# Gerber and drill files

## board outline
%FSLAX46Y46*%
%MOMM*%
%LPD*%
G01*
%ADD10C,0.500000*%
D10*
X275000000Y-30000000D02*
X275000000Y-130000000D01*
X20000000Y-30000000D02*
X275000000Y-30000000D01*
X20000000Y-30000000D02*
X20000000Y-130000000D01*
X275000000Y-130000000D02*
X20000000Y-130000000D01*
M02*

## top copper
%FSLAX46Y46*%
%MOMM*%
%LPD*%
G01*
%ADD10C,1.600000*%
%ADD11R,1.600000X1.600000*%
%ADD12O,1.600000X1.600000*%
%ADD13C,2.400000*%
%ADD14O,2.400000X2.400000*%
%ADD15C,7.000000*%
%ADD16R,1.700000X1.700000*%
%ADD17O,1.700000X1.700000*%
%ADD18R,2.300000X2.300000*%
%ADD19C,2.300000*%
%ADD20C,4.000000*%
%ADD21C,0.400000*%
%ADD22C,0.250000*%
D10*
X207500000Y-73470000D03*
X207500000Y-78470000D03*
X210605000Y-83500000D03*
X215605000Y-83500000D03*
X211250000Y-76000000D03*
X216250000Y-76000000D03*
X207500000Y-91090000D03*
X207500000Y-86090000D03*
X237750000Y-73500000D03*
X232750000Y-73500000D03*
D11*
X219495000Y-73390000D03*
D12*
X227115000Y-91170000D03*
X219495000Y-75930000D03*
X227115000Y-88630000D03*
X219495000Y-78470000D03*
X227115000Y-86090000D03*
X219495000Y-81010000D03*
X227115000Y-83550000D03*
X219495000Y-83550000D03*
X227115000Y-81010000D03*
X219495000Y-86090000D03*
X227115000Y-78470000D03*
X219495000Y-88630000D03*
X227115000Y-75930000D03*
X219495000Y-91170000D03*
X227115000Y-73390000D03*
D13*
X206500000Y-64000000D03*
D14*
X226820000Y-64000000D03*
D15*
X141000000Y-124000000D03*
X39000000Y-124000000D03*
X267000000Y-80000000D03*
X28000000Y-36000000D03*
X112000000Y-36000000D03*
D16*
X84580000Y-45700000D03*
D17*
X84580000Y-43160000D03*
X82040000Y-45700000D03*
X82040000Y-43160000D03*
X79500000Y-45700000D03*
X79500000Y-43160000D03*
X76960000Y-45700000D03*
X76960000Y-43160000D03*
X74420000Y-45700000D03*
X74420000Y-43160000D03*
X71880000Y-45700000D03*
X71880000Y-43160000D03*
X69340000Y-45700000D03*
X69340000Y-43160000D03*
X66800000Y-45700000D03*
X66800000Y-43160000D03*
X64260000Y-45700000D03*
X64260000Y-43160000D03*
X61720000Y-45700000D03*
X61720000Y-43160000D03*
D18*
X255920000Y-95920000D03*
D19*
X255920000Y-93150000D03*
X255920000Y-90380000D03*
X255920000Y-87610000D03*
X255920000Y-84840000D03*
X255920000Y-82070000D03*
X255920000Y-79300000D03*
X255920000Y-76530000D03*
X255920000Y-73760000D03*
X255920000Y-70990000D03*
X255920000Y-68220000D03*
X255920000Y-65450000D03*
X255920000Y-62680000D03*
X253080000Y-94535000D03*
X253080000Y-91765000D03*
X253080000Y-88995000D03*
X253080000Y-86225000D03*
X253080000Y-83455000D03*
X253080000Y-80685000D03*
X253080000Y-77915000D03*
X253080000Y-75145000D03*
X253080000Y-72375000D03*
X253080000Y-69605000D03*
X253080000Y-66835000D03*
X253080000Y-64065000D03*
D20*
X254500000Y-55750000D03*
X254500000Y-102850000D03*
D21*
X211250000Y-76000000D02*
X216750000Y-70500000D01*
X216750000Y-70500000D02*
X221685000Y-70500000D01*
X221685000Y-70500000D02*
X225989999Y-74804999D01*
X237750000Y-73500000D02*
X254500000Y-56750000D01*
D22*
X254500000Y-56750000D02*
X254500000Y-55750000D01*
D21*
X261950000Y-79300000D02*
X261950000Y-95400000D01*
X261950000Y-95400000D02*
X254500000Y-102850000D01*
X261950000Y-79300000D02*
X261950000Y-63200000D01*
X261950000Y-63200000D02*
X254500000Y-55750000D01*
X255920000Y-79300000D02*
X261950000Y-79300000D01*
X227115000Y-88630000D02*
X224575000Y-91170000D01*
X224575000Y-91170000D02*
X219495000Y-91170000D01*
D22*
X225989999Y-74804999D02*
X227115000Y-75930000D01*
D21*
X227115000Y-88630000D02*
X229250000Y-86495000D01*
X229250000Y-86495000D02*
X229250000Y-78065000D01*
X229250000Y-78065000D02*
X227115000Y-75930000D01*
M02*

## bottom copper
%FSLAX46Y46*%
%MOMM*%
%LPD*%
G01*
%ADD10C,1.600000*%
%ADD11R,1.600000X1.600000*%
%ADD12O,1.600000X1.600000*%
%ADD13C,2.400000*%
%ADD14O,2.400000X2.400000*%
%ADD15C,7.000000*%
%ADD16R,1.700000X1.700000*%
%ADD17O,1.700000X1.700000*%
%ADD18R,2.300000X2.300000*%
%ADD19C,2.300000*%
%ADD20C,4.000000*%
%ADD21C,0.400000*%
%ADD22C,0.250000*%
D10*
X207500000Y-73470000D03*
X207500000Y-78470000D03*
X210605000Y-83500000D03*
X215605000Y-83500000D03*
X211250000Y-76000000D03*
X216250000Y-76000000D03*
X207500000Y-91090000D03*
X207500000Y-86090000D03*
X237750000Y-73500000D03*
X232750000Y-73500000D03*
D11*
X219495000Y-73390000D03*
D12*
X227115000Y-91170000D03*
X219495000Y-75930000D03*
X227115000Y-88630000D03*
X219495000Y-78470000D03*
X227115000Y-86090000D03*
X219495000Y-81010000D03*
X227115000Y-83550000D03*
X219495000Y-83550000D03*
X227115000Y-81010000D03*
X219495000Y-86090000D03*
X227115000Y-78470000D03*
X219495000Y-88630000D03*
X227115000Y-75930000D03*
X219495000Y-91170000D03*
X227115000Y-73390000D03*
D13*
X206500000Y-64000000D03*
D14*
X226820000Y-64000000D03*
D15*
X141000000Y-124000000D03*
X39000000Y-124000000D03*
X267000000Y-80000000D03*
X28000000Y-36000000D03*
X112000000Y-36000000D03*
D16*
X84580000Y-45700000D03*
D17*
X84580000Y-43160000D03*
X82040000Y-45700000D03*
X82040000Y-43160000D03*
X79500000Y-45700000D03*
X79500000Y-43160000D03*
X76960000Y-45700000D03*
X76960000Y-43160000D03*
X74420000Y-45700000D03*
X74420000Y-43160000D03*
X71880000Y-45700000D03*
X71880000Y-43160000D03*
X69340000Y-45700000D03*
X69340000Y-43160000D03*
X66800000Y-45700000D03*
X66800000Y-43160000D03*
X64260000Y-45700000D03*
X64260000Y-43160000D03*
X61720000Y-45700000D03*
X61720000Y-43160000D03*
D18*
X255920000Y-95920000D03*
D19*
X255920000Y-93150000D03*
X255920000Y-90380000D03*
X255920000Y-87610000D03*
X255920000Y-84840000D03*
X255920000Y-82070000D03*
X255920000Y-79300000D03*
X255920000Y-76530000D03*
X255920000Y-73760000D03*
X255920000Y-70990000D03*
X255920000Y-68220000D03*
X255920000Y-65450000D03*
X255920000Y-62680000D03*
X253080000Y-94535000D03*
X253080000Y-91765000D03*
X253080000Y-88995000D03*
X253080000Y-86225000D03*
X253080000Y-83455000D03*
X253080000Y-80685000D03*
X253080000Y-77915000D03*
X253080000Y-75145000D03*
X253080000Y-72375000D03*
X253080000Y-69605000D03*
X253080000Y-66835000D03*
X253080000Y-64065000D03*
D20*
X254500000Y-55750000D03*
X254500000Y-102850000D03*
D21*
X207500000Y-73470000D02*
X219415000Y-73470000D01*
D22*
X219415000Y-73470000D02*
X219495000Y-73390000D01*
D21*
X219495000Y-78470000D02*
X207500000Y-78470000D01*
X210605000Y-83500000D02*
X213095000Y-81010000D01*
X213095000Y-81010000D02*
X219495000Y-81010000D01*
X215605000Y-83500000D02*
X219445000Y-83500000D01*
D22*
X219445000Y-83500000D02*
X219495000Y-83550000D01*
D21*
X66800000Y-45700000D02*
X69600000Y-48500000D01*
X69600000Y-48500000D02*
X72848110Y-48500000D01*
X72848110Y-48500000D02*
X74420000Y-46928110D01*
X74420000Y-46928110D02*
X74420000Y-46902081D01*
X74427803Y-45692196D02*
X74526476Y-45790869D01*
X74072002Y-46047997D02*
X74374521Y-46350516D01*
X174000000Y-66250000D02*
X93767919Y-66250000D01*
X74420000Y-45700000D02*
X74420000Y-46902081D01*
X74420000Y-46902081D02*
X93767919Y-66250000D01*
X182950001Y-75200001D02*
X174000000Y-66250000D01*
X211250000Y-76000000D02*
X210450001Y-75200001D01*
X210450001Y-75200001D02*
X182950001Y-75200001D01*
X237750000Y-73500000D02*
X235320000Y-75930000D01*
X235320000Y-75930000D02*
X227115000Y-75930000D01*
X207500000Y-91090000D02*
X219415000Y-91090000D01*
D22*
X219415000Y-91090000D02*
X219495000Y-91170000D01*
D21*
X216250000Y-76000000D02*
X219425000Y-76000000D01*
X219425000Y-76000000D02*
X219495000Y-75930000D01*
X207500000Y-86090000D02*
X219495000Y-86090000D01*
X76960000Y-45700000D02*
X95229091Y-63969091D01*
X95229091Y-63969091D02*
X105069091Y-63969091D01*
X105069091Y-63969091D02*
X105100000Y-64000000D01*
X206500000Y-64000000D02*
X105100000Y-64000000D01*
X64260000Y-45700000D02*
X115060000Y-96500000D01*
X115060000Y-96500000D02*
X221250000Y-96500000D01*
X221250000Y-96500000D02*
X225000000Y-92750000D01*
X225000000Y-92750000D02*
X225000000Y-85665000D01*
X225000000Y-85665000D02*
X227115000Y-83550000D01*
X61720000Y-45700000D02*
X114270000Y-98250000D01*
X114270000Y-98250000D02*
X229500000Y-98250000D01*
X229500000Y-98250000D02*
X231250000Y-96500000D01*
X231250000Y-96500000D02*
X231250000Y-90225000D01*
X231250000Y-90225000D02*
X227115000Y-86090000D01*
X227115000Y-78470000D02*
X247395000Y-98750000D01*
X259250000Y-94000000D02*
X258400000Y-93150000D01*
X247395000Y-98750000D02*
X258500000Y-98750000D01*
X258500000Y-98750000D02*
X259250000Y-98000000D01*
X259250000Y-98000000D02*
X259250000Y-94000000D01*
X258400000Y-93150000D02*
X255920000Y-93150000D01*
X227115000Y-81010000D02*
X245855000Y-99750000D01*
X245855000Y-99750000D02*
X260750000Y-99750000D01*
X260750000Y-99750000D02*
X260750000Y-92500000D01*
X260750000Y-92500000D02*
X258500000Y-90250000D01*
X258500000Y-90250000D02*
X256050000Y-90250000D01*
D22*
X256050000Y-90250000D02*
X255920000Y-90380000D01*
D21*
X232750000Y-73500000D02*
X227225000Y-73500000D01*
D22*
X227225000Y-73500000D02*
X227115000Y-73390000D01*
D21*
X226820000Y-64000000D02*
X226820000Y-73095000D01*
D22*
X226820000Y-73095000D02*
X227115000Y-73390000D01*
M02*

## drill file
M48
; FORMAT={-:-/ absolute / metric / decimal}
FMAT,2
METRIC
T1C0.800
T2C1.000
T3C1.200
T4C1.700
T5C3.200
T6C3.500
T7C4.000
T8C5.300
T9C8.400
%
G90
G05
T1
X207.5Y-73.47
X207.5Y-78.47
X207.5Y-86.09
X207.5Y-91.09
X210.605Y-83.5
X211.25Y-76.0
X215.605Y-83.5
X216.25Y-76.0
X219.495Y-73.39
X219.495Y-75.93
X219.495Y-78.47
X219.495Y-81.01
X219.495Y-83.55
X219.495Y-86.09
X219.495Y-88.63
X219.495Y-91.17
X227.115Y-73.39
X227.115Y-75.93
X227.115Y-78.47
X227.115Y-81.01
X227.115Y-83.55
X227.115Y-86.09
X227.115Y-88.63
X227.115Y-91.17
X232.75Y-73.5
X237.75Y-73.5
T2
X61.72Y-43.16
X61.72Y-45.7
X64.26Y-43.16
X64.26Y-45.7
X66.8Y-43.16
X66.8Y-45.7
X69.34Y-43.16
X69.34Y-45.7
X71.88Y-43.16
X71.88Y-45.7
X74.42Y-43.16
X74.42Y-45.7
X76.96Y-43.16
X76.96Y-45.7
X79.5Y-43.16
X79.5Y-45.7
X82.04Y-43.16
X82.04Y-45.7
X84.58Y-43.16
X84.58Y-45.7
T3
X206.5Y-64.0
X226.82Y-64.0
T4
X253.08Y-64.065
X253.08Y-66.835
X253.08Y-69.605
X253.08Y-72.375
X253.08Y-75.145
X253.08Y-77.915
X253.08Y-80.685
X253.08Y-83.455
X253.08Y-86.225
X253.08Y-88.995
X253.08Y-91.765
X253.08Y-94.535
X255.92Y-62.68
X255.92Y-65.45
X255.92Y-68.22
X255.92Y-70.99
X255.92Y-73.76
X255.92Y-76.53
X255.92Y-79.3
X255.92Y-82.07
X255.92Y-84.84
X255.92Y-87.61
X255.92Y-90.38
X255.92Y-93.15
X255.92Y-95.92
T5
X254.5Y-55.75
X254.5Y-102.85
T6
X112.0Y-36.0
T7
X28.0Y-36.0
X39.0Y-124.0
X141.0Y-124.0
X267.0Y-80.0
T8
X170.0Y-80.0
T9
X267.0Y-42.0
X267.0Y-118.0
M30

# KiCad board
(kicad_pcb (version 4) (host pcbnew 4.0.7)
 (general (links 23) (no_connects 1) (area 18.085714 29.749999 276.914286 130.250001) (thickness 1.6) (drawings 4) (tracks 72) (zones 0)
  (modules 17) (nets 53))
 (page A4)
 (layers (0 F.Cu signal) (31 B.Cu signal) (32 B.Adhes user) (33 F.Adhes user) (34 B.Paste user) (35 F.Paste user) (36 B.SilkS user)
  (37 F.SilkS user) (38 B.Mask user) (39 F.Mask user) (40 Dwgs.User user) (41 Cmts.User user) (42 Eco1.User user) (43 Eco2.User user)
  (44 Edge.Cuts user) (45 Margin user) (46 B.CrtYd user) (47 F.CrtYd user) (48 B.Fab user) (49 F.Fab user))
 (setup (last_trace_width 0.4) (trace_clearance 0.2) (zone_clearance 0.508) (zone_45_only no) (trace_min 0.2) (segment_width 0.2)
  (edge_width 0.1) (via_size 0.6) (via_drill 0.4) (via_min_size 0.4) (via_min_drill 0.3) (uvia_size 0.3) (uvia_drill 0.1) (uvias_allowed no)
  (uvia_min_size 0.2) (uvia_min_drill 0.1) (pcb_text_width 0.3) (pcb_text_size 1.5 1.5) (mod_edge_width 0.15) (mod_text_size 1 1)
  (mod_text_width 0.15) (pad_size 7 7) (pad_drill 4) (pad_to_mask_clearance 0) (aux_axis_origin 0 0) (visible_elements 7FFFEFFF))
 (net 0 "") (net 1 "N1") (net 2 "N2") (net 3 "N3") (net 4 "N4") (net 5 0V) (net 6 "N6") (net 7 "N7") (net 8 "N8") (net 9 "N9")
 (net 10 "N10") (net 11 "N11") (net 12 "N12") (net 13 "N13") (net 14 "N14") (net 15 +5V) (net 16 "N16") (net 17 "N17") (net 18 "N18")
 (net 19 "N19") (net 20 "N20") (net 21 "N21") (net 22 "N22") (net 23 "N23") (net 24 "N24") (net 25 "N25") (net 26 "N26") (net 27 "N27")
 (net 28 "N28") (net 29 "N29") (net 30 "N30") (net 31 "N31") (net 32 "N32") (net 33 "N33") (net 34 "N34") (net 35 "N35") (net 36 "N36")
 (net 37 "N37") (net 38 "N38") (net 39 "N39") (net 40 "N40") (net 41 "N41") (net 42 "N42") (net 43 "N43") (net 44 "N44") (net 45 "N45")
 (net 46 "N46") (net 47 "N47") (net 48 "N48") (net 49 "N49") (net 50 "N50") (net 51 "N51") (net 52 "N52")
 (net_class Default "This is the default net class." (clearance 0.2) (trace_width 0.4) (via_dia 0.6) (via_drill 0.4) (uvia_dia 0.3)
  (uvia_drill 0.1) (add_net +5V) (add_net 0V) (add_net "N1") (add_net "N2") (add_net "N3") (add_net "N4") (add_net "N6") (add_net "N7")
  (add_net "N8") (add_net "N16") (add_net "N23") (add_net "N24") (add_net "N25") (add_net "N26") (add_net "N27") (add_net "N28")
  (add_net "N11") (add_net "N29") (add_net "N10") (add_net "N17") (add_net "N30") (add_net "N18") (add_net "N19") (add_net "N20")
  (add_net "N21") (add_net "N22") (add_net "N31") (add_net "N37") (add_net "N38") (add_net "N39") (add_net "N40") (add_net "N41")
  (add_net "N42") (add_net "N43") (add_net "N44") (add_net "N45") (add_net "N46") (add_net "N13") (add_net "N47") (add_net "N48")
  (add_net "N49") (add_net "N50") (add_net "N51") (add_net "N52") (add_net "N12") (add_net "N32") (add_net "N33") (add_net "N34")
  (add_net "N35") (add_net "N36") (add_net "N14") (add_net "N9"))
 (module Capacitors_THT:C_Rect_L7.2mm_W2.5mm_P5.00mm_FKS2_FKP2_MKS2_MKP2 (layer F.Cu) (at 207.5 73.47 270)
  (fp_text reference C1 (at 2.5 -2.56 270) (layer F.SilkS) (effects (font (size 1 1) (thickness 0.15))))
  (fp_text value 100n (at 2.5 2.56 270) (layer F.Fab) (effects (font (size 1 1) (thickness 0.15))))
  (pad 1 thru_hole circle (at 0 0 270) (size 1.6 1.6) (drill 0.8) (layers *.Cu *.Mask) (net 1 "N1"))
  (pad 2 thru_hole circle (at 5 0 270) (size 1.6 1.6) (drill 0.8) (layers *.Cu *.Mask) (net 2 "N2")))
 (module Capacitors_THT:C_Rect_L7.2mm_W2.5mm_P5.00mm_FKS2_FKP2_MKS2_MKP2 (layer F.Cu) (at 210.605 83.5)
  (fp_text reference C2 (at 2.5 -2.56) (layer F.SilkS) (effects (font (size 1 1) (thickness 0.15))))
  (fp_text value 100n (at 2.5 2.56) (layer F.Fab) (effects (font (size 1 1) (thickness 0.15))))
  (pad 1 thru_hole circle (at 0 0) (size 1.6 1.6) (drill 0.8) (layers *.Cu *.Mask) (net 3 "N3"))
  (pad 2 thru_hole circle (at 5 0) (size 1.6 1.6) (drill 0.8) (layers *.Cu *.Mask) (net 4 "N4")))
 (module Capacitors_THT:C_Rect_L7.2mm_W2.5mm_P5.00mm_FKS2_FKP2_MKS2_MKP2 (layer F.Cu) (at 211.25 76)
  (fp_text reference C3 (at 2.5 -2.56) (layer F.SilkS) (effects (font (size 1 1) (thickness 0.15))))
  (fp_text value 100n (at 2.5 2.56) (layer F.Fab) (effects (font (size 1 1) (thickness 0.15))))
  (pad 1 thru_hole circle (at 0 0) (size 1.6 1.6) (drill 0.8) (layers *.Cu *.Mask) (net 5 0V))
  (pad 2 thru_hole circle (at 5 0) (size 1.6 1.6) (drill 0.8) (layers *.Cu *.Mask) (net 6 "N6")))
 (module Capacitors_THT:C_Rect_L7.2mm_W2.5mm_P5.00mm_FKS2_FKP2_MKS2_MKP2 (layer F.Cu) (at 207.5 91.09 90)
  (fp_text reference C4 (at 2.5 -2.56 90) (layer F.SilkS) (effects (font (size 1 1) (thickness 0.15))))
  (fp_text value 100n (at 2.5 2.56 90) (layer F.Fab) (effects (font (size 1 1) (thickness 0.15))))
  (pad 1 thru_hole circle (at 0 0 90) (size 1.6 1.6) (drill 0.8) (layers *.Cu *.Mask) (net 5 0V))
  (pad 2 thru_hole circle (at 5 0 90) (size 1.6 1.6) (drill 0.8) (layers *.Cu *.Mask) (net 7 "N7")))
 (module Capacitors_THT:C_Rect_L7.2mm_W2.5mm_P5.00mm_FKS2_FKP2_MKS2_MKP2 (layer F.Cu) (at 237.75 73.5 180)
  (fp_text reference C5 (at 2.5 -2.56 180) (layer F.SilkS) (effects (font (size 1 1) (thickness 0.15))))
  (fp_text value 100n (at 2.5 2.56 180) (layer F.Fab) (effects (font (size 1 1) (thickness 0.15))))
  (pad 1 thru_hole circle (at 0 0 180) (size 1.6 1.6) (drill 0.8) (layers *.Cu *.Mask) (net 5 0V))
  (pad 2 thru_hole circle (at 5 0 180) (size 1.6 1.6) (drill 0.8) (layers *.Cu *.Mask) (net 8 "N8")))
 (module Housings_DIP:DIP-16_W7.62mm (layer F.Cu) (at 219.495 73.39)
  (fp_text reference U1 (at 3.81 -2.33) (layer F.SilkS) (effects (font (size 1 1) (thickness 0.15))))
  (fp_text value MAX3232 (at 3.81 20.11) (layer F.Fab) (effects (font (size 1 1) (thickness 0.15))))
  (pad 1 thru_hole rect (at 0 0) (size 1.6 1.6) (drill 0.8) (layers *.Cu *.Mask) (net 1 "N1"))
  (pad 9 thru_hole oval (at 7.62 17.78) (size 1.6 1.6) (drill 0.8) (layers *.Cu *.Mask) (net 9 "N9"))
  (pad 2 thru_hole oval (at 0 2.54) (size 1.6 1.6) (drill 0.8) (layers *.Cu *.Mask) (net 6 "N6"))
  (pad 10 thru_hole oval (at 7.62 15.24) (size 1.6 1.6) (drill 0.8) (layers *.Cu *.Mask) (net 5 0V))
  (pad 3 thru_hole oval (at 0 5.08) (size 1.6 1.6) (drill 0.8) (layers *.Cu *.Mask) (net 2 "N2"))
  (pad 11 thru_hole oval (at 7.62 12.7) (size 1.6 1.6) (drill 0.8) (layers *.Cu *.Mask) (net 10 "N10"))
  (pad 4 thru_hole oval (at 0 7.62) (size 1.6 1.6) (drill 0.8) (layers *.Cu *.Mask) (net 3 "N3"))
  (pad 12 thru_hole oval (at 7.62 10.16) (size 1.6 1.6) (drill 0.8) (layers *.Cu *.Mask) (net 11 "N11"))
  (pad 5 thru_hole oval (at 0 10.16) (size 1.6 1.6) (drill 0.8) (layers *.Cu *.Mask) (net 4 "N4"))
  (pad 13 thru_hole oval (at 7.62 7.62) (size 1.6 1.6) (drill 0.8) (layers *.Cu *.Mask) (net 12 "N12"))
  (pad 6 thru_hole oval (at 0 12.7) (size 1.6 1.6) (drill 0.8) (layers *.Cu *.Mask) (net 7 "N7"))
  (pad 14 thru_hole oval (at 7.62 5.08) (size 1.6 1.6) (drill 0.8) (layers *.Cu *.Mask) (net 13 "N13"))
  (pad 7 thru_hole oval (at 0 15.24) (size 1.6 1.6) (drill 0.8) (layers *.Cu *.Mask) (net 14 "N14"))
  (pad 15 thru_hole oval (at 7.62 2.54) (size 1.6 1.6) (drill 0.8) (layers *.Cu *.Mask) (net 5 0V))
  (pad 8 thru_hole oval (at 0 17.78) (size 1.6 1.6) (drill 0.8) (layers *.Cu *.Mask) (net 5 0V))
  (pad 16 thru_hole oval (at 7.62 0) (size 1.6 1.6) (drill 0.8) (layers *.Cu *.Mask) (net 8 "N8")))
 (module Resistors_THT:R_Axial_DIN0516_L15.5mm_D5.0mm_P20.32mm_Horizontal (layer F.Cu) (at 206.5 64)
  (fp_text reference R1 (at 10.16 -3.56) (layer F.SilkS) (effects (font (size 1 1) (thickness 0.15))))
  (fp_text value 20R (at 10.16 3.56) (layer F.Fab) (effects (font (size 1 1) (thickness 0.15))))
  (pad 1 thru_hole circle (at 0 0) (size 2.4 2.4) (drill 1.2) (layers *.Cu *.Mask) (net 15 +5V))
  (pad 2 thru_hole oval (at 20.32 0) (size 2.4 2.4) (drill 1.2) (layers *.Cu *.Mask) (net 8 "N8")))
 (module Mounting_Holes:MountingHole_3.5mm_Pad (layer F.Cu) (at 141 124)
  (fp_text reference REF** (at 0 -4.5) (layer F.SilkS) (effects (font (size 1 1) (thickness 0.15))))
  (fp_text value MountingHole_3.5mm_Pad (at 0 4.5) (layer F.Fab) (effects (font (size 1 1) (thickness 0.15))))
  (pad 1 thru_hole circle (at 0 0) (size 7 7) (drill 4) (layers *.Cu *.Mask)))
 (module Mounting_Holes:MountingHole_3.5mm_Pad (layer F.Cu) (at 40 124)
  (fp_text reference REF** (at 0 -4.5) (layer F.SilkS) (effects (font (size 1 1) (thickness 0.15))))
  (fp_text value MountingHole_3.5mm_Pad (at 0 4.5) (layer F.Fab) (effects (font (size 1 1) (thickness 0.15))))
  (pad 1 thru_hole circle (at -1 0) (size 7 7) (drill 4) (layers *.Cu *.Mask)))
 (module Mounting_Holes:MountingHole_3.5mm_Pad (layer F.Cu) (at 267 80)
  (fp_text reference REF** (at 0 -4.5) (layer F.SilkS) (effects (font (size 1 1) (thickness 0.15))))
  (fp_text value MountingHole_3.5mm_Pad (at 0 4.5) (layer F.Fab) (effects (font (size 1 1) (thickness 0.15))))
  (pad 1 thru_hole circle (at 0 0) (size 7 7) (drill 4) (layers *.Cu *.Mask)))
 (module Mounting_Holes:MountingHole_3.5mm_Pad (layer F.Cu) (at 28 36)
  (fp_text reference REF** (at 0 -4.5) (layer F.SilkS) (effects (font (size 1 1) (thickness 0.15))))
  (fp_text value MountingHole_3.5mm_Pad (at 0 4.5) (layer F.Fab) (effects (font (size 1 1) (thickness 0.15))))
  (pad 1 thru_hole circle (at 0 0) (size 7 7) (drill 4) (layers *.Cu *.Mask)))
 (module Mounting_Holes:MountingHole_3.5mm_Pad (layer F.Cu) (at 112 36)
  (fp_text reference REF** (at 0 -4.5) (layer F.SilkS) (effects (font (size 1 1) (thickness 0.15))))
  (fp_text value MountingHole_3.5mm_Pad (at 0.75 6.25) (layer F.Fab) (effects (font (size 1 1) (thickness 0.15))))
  (pad 1 thru_hole circle (at 0 0) (size 7 7) (drill 3.5) (layers *.Cu *.Mask)))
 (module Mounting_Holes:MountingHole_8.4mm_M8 (layer F.Cu) (at 267 42)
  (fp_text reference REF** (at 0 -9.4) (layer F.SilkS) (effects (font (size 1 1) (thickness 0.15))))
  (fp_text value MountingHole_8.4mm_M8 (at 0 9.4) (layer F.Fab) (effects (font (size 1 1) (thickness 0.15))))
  (pad 1 np_thru_hole circle (at 0 0) (size 8.4 8.4) (drill 8.4) (layers *.Cu *.Mask)))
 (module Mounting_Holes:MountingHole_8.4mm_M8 (layer F.Cu) (at 267 118)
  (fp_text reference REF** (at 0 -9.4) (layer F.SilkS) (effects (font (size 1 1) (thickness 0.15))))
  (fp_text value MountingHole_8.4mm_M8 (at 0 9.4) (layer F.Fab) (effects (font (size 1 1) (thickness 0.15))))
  (pad 1 np_thru_hole circle (at 0 0) (size 8.4 8.4) (drill 8.4) (layers *.Cu *.Mask)))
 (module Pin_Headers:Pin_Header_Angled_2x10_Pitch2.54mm (layer B.Cu) (at 84.58 45.7 90)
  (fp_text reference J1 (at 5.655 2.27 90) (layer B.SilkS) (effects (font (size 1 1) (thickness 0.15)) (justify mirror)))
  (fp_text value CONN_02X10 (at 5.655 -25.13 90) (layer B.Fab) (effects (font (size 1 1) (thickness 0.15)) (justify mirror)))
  (pad 1 thru_hole rect (at 0 0 90) (size 1.7 1.7) (drill 1) (layers *.Cu *.Mask) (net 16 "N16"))
  (pad 2 thru_hole oval (at 2.54 0 90) (size 1.7 1.7) (drill 1) (layers *.Cu *.Mask) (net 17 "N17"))
  (pad 3 thru_hole oval (at 0 -2.54 90) (size 1.7 1.7) (drill 1) (layers *.Cu *.Mask) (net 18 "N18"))
  (pad 4 thru_hole oval (at 2.54 -2.54 90) (size 1.7 1.7) (drill 1) (layers *.Cu *.Mask) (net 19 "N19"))
  (pad 5 thru_hole oval (at 0 -5.08 90) (size 1.7 1.7) (drill 1) (layers *.Cu *.Mask) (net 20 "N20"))
  (pad 6 thru_hole oval (at 2.54 -5.08 90) (size 1.7 1.7) (drill 1) (layers *.Cu *.Mask) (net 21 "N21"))
  (pad 7 thru_hole oval (at 0 -7.62 90) (size 1.7 1.7) (drill 1) (layers *.Cu *.Mask) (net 15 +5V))
  (pad 8 thru_hole oval (at 2.54 -7.62 90) (size 1.7 1.7) (drill 1) (layers *.Cu *.Mask) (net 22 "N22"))
  (pad 9 thru_hole oval (at 0 -10.16 90) (size 1.7 1.7) (drill 1) (layers *.Cu *.Mask) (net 5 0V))
  (pad 10 thru_hole oval (at 2.54 -10.16 90) (size 1.7 1.7) (drill 1) (layers *.Cu *.Mask) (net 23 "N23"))
  (pad 11 thru_hole oval (at 0 -12.7 90) (size 1.7 1.7) (drill 1) (layers *.Cu *.Mask) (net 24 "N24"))
  (pad 12 thru_hole oval (at 2.54 -12.7 90) (size 1.7 1.7) (drill 1) (layers *.Cu *.Mask) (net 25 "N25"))
  (pad 13 thru_hole oval (at 0 -15.24 90) (size 1.7 1.7) (drill 1) (layers *.Cu *.Mask) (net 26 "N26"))
  (pad 14 thru_hole oval (at 2.54 -15.24 90) (size 1.7 1.7) (drill 1) (layers *.Cu *.Mask) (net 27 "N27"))
  (pad 15 thru_hole oval (at 0 -17.78 90) (size 1.7 1.7) (drill 1) (layers *.Cu *.Mask) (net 5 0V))
  (pad 16 thru_hole oval (at 2.54 -17.78 90) (size 1.7 1.7) (drill 1) (layers *.Cu *.Mask) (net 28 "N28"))
  (pad 17 thru_hole oval (at 0 -20.32 90) (size 1.7 1.7) (drill 1) (layers *.Cu *.Mask) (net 11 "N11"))
  (pad 18 thru_hole oval (at 2.54 -20.32 90) (size 1.7 1.7) (drill 1) (layers *.Cu *.Mask) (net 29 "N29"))
  (pad 19 thru_hole oval (at 0 -22.86 90) (size 1.7 1.7) (drill 1) (layers *.Cu *.Mask) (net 10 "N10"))
  (pad 20 thru_hole oval (at 2.54 -22.86 90) (size 1.7 1.7) (drill 1) (layers *.Cu *.Mask) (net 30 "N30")))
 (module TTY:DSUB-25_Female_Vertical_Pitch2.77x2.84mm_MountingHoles (layer F.Cu) (at 255.92 95.92 270)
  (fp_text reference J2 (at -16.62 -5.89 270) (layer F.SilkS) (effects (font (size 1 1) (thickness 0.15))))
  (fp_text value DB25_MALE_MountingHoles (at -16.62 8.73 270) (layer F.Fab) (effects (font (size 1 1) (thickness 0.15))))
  (pad 1 thru_hole rect (at 0 0 270) (size 2.3 2.3) (drill 1.7) (layers *.Cu *.Mask) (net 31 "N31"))
  (pad 2 thru_hole circle (at -2.77 0 270) (size 2.3 2.3) (drill 1.7) (layers *.Cu *.Mask) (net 13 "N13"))
  (pad 3 thru_hole circle (at -5.54 0 270) (size 2.3 2.3) (drill 1.7) (layers *.Cu *.Mask) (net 12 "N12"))
  (pad 4 thru_hole circle (at -8.31 0 270) (size 2.3 2.3) (drill 1.7) (layers *.Cu *.Mask) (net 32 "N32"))
  (pad 5 thru_hole circle (at -11.08 0 270) (size 2.3 2.3) (drill 1.7) (layers *.Cu *.Mask) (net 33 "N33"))
  (pad 6 thru_hole circle (at -13.85 0 270) (size 2.3 2.3) (drill 1.7) (layers *.Cu *.Mask) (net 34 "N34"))
  (pad 7 thru_hole circle (at -16.62 0 270) (size 2.3 2.3) (drill 1.7) (layers *.Cu *.Mask) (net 5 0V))
  (pad 8 thru_hole circle (at -19.39 0 270) (size 2.3 2.3) (drill 1.7) (layers *.Cu *.Mask) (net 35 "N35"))
  (pad 9 thru_hole circle (at -22.16 0 270) (size 2.3 2.3) (drill 1.7) (layers *.Cu *.Mask) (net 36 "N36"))
  (pad 10 thru_hole circle (at -24.93 0 270) (size 2.3 2.3) (drill 1.7) (layers *.Cu *.Mask) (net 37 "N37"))
  (pad 11 thru_hole circle (at -27.7 0 270) (size 2.3 2.3) (drill 1.7) (layers *.Cu *.Mask) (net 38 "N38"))
  (pad 12 thru_hole circle (at -30.47 0 270) (size 2.3 2.3) (drill 1.7) (layers *.Cu *.Mask) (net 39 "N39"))
  (pad 13 thru_hole circle (at -33.24 0 270) (size 2.3 2.3) (drill 1.7) (layers *.Cu *.Mask) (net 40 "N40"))
  (pad 14 thru_hole circle (at -1.385 2.84 270) (size 2.3 2.3) (drill 1.7) (layers *.Cu *.Mask) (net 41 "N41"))
  (pad 15 thru_hole circle (at -4.155 2.84 270) (size 2.3 2.3) (drill 1.7) (layers *.Cu *.Mask) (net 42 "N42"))
  (pad 16 thru_hole circle (at -6.925 2.84 270) (size 2.3 2.3) (drill 1.7) (layers *.Cu *.Mask) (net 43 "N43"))
  (pad 17 thru_hole circle (at -9.695 2.84 270) (size 2.3 2.3) (drill 1.7) (layers *.Cu *.Mask) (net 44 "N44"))
  (pad 18 thru_hole circle (at -12.465 2.84 270) (size 2.3 2.3) (drill 1.7) (layers *.Cu *.Mask) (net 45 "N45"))
  (pad 19 thru_hole circle (at -15.235 2.84 270) (size 2.3 2.3) (drill 1.7) (layers *.Cu *.Mask) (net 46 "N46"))
  (pad 20 thru_hole circle (at -18.005 2.84 270) (size 2.3 2.3) (drill 1.7) (layers *.Cu *.Mask) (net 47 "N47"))
  (pad 21 thru_hole circle (at -20.775 2.84 270) (size 2.3 2.3) (drill 1.7) (layers *.Cu *.Mask) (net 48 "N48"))
  (pad 22 thru_hole circle (at -23.545 2.84 270) (size 2.3 2.3) (drill 1.7) (layers *.Cu *.Mask) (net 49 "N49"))
  (pad 23 thru_hole circle (at -26.315 2.84 270) (size 2.3 2.3) (drill 1.7) (layers *.Cu *.Mask) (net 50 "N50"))
  (pad 24 thru_hole circle (at -29.085 2.84 270) (size 2.3 2.3) (drill 1.7) (layers *.Cu *.Mask) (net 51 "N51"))
  (pad 25 thru_hole circle (at -31.855 2.84 270) (size 2.3 2.3) (drill 1.7) (layers *.Cu *.Mask) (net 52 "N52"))
  (pad 0 thru_hole circle (at -40.17 1.42 270) (size 4 4) (drill 3.2) (layers *.Cu *.Mask) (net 5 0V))
  (pad 0 thru_hole circle (at 6.93 1.42 270) (size 4 4) (drill 3.2) (layers *.Cu *.Mask) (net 5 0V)))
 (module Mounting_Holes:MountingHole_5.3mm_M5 (layer F.Cu) (at 170 80)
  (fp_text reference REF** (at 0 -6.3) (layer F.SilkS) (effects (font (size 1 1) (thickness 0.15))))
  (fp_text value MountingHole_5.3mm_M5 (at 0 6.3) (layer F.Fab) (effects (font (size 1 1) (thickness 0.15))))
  (pad "" np_thru_hole circle (at 0 0) (size 5.3 5.3) (drill 5.3) (layers *.Cu *.Mask F.Paste)))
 (gr_line (start 275 30) (end 275 130) (layer Edge.Cuts) (width 0.5))
 (gr_line (start 20 30) (end 275 30) (layer Edge.Cuts) (width 0.5))
 (gr_line (start 20 30) (end 20 130) (layer Edge.Cuts) (width 0.5))
 (gr_line (start 275 130) (end 20 130) (layer Edge.Cuts) (width 0.5))
 (segment (start 207.5 73.47) (end 219.415 73.47) (width 0.4) (layer B.Cu) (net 1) (status 30))
 (segment (start 219.415 73.47) (end 219.495 73.39) (width 0.25) (layer B.Cu) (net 1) (status 30))
 (segment (start 219.495 78.47) (end 207.5 78.47) (width 0.4) (layer B.Cu) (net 2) (status 30))
 (segment (start 210.605 83.5) (end 213.095 81.01) (width 0.4) (layer B.Cu) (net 3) (status 10))
 (segment (start 213.095 81.01) (end 219.495 81.01) (width 0.4) (layer B.Cu) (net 3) (status 20))
 (segment (start 215.605 83.5) (end 219.445 83.5) (width 0.4) (layer B.Cu) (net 4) (status 30))
 (segment (start 219.445 83.5) (end 219.495 83.55) (width 0.25) (layer B.Cu) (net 4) (status 30))
 (segment (start 66.8 45.7) (end 69.6 48.5) (width 0.4) (layer B.Cu) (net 5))
 (segment (start 69.6 48.5) (end 72.84811 48.5) (width 0.4) (layer B.Cu) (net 5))
 (segment (start 72.84811 48.5) (end 74.42 46.92811) (width 0.4) (layer B.Cu) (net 5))
 (segment (start 74.42 46.92811) (end 74.42 46.902081) (width 0.4) (layer B.Cu) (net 5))
 (segment (start 74.427803 45.692196) (end 74.526476 45.790869) (width 0.4) (layer B.Cu) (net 5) (status 30))
 (segment (start 74.072002 46.047997) (end 74.374521 46.350516) (width 0.4) (layer B.Cu) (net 5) (status 30))
 (segment (start 174 66.25) (end 93.767919 66.25) (width 0.4) (layer B.Cu) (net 5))
 (segment (start 74.42 45.7) (end 74.42 46.902081) (width 0.4) (layer B.Cu) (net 5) (status 10))
 (segment (start 74.42 46.902081) (end 93.767919 66.25) (width 0.4) (layer B.Cu) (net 5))
 (segment (start 211.25 76) (end 216.75 70.5) (width 0.4) (layer F.Cu) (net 5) (status 10))
 (segment (start 216.75 70.5) (end 221.685 70.5) (width 0.4) (layer F.Cu) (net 5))
 (segment (start 221.685 70.5) (end 225.989999 74.804999) (width 0.4) (layer F.Cu) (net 5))
 (segment (start 182.950001 75.200001) (end 174 66.25) (width 0.4) (layer B.Cu) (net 5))
 (segment (start 211.25 76) (end 210.450001 75.200001) (width 0.4) (layer B.Cu) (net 5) (status 10))
 (segment (start 210.450001 75.200001) (end 182.950001 75.200001) (width 0.4) (layer B.Cu) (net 5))
 (segment (start 237.75 73.5) (end 254.5 56.75) (width 0.4) (layer F.Cu) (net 5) (status 30))
 (segment (start 254.5 56.75) (end 254.5 55.75) (width 0.25) (layer F.Cu) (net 5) (status 30))
 (segment (start 261.95 79.3) (end 261.95 95.4) (width 0.4) (layer F.Cu) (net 5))
 (segment (start 261.95 95.4) (end 254.5 102.85) (width 0.4) (layer F.Cu) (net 5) (status 20))
 (segment (start 261.95 79.3) (end 261.95 63.2) (width 0.4) (layer F.Cu) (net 5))
 (segment (start 261.95 63.2) (end 254.5 55.75) (width 0.4) (layer F.Cu) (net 5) (status 20))
 (segment (start 255.92 79.3) (end 261.95 79.3) (width 0.4) (layer F.Cu) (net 5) (status 10))
 (segment (start 227.115 88.63) (end 224.575 91.17) (width 0.4) (layer F.Cu) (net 5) (status 10))
 (segment (start 224.575 91.17) (end 219.495 91.17) (width 0.4) (layer F.Cu) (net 5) (status 20))
 (segment (start 225.989999 74.804999) (end 227.115 75.93) (width 0.25) (layer F.Cu) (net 5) (status 20))
 (segment (start 237.75 73.5) (end 235.32 75.93) (width 0.4) (layer B.Cu) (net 5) (status 10))
 (segment (start 235.32 75.93) (end 227.115 75.93) (width 0.4) (layer B.Cu) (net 5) (status 20))
 (segment (start 227.115 88.63) (end 229.25 86.495) (width 0.4) (layer F.Cu) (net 5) (status 10))
 (segment (start 229.25 86.495) (end 229.25 78.065) (width 0.4) (layer F.Cu) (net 5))
 (segment (start 229.25 78.065) (end 227.115 75.93) (width 0.4) (layer F.Cu) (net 5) (status 20))
 (segment (start 207.5 91.09) (end 219.415 91.09) (width 0.4) (layer B.Cu) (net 5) (status 30))
 (segment (start 219.415 91.09) (end 219.495 91.17) (width 0.25) (layer B.Cu) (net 5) (status 30))
 (segment (start 216.25 76) (end 219.425 76) (width 0.4) (layer B.Cu) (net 6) (status 30))
 (segment (start 219.425 76) (end 219.495 75.93) (width 0.4) (layer B.Cu) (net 6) (status 30))
 (segment (start 207.5 86.09) (end 219.495 86.09) (width 0.4) (layer B.Cu) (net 7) (status 30))
 (segment (start 76.96 45.7) (end 95.229091 63.969091) (width 0.4) (layer B.Cu) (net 15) (status 10))
 (segment (start 95.229091 63.969091) (end 105.069091 63.969091) (width 0.4) (layer B.Cu) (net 15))
 (segment (start 105.069091 63.969091) (end 105.1 64) (width 0.4) (layer B.Cu) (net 15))
 (segment (start 206.5 64) (end 105.1 64) (width 0.4) (layer B.Cu) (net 15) (status 10))
 (segment (start 64.26 45.7) (end 115.06 96.5) (width 0.4) (layer B.Cu) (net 11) (status 10))
 (segment (start 115.06 96.5) (end 221.25 96.5) (width 0.4) (layer B.Cu) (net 11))
 (segment (start 221.25 96.5) (end 225 92.75) (width 0.4) (layer B.Cu) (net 11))
 (segment (start 225 92.75) (end 225 85.665) (width 0.4) (layer B.Cu) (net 11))
 (segment (start 225 85.665) (end 227.115 83.55) (width 0.4) (layer B.Cu) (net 11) (status 20))
 (segment (start 61.72 45.7) (end 114.27 98.25) (width 0.4) (layer B.Cu) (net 10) (status 10))
 (segment (start 114.27 98.25) (end 229.5 98.25) (width 0.4) (layer B.Cu) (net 10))
 (segment (start 229.5 98.25) (end 231.25 96.5) (width 0.4) (layer B.Cu) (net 10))
 (segment (start 231.25 96.5) (end 231.25 90.225) (width 0.4) (layer B.Cu) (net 10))
 (segment (start 231.25 90.225) (end 227.115 86.09) (width 0.4) (layer B.Cu) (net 10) (status 20))
 (segment (start 227.115 78.47) (end 247.395 98.75) (width 0.4) (layer B.Cu) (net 13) (status 10))
 (segment (start 259.25 94) (end 258.4 93.15) (width 0.4) (layer B.Cu) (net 13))
 (segment (start 247.395 98.75) (end 258.5 98.75) (width 0.4) (layer B.Cu) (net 13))
 (segment (start 258.5 98.75) (end 259.25 98) (width 0.4) (layer B.Cu) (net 13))
 (segment (start 259.25 98) (end 259.25 94) (width 0.4) (layer B.Cu) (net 13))
 (segment (start 258.4 93.15) (end 255.92 93.15) (width 0.4) (layer B.Cu) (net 13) (status 20))
 (segment (start 227.115 81.01) (end 245.855 99.75) (width 0.4) (layer B.Cu) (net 12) (status 10))
 (segment (start 245.855 99.75) (end 260.75 99.75) (width 0.4) (layer B.Cu) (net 12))
 (segment (start 260.75 99.75) (end 260.75 92.5) (width 0.4) (layer B.Cu) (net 12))
 (segment (start 260.75 92.5) (end 258.5 90.25) (width 0.4) (layer B.Cu) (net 12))
 (segment (start 258.5 90.25) (end 256.05 90.25) (width 0.4) (layer B.Cu) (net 12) (status 20))
 (segment (start 256.05 90.25) (end 255.92 90.38) (width 0.25) (layer B.Cu) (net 12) (status 30))
 (segment (start 232.75 73.5) (end 227.225 73.5) (width 0.4) (layer B.Cu) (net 8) (status 30))
 (segment (start 227.225 73.5) (end 227.115 73.39) (width 0.25) (layer B.Cu) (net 8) (status 30))
 (segment (start 226.82 64) (end 226.82 73.095) (width 0.4) (layer B.Cu) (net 8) (status 30))
 (segment (start 226.82 73.095) (end 227.115 73.39) (width 0.25) (layer B.Cu) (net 8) (status 30)))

